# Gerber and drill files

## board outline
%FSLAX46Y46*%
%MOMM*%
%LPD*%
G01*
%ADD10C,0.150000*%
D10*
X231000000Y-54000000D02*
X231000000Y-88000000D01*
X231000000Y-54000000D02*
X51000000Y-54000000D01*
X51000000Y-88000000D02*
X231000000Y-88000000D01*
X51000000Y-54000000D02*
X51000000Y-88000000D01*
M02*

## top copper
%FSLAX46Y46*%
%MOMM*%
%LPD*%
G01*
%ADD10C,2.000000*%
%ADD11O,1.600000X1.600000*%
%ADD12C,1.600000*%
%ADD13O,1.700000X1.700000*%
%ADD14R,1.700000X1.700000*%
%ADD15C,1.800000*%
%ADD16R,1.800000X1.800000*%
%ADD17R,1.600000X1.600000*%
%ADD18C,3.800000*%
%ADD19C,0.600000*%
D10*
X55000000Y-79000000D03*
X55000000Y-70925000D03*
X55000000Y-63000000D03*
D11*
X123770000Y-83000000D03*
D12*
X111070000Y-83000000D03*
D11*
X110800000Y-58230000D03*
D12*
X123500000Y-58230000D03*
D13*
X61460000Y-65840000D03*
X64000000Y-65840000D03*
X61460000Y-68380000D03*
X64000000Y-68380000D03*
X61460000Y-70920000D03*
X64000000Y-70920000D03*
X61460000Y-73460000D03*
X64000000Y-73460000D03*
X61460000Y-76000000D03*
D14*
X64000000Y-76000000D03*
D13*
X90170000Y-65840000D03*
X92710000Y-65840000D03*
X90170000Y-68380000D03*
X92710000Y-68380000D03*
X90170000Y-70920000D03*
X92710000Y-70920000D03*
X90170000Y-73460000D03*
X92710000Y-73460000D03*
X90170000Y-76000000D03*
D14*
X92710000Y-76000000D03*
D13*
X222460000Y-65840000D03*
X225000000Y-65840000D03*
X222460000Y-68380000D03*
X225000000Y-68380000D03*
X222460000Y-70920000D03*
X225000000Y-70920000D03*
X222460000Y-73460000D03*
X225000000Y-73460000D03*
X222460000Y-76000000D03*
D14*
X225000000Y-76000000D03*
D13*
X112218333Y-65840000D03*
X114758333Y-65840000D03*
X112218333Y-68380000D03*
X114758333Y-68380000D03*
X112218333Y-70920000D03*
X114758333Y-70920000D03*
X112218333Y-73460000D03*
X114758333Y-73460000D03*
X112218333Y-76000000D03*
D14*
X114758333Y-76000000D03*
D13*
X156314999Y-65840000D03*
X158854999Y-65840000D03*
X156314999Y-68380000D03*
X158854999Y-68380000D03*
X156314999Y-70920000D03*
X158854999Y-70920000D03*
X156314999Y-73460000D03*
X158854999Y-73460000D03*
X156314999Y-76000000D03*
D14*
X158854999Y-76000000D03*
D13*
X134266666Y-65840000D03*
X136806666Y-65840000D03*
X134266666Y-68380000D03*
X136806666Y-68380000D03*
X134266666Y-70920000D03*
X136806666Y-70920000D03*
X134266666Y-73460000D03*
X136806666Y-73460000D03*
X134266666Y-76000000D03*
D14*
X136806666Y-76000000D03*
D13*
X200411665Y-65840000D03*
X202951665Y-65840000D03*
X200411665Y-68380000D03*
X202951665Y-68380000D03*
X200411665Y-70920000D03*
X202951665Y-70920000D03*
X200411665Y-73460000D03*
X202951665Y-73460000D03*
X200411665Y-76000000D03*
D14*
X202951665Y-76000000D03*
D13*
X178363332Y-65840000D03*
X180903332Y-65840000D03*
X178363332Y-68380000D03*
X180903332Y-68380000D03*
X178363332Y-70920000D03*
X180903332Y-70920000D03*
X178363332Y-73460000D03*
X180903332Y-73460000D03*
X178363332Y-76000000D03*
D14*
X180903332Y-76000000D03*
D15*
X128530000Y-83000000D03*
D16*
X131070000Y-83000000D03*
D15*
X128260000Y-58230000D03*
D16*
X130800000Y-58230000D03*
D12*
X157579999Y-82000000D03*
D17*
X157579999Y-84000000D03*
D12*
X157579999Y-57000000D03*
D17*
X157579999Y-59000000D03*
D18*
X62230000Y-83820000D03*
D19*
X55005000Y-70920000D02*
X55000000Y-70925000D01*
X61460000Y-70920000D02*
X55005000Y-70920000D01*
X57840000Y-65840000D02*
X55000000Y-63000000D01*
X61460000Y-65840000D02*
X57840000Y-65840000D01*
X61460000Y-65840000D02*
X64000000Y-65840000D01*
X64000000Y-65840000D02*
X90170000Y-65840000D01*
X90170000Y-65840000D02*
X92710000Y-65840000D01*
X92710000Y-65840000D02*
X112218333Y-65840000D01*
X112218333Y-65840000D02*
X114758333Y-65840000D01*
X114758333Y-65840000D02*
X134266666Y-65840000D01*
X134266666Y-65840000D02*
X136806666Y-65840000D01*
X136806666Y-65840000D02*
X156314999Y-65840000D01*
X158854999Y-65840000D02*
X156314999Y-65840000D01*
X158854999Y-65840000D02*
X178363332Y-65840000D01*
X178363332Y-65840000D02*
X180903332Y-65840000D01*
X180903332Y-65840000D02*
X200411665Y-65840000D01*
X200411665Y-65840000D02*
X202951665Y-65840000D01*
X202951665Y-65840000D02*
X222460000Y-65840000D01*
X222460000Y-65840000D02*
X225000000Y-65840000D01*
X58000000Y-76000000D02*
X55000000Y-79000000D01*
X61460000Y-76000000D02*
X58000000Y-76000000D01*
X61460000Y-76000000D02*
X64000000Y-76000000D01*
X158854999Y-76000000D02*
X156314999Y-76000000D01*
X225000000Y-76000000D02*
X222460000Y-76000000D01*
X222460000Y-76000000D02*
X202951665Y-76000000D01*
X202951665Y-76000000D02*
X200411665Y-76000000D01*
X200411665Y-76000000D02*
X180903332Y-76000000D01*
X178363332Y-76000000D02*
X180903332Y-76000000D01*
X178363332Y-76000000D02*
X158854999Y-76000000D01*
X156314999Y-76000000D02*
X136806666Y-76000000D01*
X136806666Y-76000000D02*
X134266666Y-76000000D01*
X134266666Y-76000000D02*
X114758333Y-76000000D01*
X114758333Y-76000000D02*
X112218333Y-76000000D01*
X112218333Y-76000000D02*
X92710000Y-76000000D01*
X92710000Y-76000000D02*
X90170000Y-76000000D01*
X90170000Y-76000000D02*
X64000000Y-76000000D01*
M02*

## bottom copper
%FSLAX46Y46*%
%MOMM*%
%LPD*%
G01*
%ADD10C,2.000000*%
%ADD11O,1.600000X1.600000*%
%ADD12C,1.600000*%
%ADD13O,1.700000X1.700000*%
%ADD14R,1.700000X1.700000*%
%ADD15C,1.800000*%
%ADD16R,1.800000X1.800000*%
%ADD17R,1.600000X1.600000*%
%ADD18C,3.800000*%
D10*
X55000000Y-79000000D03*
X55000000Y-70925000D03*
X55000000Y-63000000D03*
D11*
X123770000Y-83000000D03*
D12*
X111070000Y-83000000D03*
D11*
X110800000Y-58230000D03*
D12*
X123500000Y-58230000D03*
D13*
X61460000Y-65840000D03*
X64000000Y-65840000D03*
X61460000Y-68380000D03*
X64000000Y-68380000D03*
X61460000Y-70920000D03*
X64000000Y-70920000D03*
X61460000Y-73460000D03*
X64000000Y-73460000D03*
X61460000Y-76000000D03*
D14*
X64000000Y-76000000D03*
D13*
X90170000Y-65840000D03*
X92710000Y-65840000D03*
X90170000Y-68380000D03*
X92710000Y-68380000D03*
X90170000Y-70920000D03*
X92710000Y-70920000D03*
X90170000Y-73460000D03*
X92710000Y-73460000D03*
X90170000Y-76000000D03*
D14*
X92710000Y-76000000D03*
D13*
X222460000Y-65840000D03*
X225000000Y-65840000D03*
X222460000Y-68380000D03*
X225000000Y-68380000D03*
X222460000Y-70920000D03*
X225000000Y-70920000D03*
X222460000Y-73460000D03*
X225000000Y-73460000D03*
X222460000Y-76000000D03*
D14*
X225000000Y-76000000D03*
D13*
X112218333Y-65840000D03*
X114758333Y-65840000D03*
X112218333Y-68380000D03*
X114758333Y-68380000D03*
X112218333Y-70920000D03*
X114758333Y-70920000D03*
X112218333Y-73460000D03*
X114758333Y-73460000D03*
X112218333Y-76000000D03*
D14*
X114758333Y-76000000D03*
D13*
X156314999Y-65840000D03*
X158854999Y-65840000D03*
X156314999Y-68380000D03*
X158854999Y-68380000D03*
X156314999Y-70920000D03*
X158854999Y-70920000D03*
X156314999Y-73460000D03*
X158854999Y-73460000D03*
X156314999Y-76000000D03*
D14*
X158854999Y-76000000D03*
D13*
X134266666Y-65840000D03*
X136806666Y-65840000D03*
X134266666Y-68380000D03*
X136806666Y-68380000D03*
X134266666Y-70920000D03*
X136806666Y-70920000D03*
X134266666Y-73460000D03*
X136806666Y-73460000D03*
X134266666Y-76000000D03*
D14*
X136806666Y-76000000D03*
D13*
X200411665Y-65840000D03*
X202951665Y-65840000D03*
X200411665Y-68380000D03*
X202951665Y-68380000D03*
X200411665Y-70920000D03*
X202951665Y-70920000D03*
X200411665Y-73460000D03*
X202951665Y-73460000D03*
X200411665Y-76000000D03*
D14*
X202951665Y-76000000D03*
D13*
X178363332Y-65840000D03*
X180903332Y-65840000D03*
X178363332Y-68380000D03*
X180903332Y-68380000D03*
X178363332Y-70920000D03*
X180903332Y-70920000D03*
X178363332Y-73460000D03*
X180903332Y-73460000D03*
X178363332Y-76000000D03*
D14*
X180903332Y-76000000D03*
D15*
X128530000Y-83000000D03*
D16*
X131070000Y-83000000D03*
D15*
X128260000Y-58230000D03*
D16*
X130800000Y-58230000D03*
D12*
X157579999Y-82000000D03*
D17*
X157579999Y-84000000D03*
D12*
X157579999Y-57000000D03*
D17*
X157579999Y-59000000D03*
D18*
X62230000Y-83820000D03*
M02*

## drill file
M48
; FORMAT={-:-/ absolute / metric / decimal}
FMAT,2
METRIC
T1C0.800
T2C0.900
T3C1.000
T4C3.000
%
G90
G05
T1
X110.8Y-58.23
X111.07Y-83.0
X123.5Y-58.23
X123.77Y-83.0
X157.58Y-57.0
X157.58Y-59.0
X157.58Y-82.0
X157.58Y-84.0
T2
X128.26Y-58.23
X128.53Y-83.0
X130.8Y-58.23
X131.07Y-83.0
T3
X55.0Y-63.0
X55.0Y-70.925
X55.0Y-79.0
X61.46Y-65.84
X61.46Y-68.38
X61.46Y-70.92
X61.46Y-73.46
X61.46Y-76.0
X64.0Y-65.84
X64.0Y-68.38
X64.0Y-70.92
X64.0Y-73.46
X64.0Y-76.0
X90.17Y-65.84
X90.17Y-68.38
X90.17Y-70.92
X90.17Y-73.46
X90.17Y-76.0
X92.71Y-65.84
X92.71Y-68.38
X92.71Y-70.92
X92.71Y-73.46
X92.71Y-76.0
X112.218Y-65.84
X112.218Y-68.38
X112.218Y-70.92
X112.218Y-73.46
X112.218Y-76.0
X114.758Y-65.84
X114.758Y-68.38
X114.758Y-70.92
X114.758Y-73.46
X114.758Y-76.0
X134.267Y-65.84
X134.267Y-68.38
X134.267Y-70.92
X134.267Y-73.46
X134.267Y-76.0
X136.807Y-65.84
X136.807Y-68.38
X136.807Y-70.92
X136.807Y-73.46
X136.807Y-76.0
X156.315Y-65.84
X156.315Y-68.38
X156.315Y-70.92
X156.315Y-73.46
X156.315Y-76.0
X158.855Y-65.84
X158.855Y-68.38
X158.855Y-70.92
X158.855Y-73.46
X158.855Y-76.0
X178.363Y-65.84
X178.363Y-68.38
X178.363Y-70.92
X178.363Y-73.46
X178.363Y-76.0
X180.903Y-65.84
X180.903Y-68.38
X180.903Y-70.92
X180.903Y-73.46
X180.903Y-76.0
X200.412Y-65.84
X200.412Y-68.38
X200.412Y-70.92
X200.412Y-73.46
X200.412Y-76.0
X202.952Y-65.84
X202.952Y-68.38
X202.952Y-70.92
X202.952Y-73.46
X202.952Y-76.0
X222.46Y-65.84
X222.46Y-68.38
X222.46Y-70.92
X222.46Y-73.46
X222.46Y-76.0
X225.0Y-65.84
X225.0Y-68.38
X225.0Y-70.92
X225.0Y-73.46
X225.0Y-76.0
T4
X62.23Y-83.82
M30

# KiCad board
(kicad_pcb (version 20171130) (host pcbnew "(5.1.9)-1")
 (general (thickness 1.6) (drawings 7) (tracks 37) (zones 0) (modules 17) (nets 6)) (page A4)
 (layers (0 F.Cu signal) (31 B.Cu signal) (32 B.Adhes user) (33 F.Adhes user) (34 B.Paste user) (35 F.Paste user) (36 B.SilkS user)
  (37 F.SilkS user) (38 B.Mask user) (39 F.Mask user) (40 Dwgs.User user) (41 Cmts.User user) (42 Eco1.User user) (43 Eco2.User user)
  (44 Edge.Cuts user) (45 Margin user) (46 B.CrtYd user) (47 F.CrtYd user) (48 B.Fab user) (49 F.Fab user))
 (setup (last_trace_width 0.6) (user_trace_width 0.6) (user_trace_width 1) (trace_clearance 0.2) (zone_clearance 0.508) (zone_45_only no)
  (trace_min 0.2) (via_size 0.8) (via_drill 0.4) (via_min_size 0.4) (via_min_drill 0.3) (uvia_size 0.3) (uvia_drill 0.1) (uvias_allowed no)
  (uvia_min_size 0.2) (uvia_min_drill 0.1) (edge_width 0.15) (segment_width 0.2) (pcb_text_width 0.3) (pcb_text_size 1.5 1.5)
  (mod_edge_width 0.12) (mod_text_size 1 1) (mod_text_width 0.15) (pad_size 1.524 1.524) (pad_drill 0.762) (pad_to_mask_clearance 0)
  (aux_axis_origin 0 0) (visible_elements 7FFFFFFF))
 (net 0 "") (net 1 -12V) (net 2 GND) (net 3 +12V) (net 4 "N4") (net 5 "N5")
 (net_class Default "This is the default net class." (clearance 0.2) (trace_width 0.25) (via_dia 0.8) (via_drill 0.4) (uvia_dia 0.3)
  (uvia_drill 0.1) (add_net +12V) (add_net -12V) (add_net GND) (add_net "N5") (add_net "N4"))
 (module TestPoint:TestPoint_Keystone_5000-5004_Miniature (layer F.Cu) (at 55 79)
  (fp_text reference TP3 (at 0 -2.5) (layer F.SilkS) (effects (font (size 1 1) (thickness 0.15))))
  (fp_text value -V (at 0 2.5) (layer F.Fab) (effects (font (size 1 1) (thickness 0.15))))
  (pad 1 thru_hole circle (at 0 0) (size 2 2) (drill 1) (layers *.Cu *.Mask) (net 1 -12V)))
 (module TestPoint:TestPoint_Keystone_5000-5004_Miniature (layer F.Cu) (at 55 70.925)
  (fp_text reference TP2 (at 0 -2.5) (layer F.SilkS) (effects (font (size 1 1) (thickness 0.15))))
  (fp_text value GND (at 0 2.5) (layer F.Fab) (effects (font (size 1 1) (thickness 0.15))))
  (pad 1 thru_hole circle (at 0 0) (size 2 2) (drill 1) (layers *.Cu *.Mask) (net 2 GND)))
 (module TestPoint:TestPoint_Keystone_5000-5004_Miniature (layer F.Cu) (at 55 63)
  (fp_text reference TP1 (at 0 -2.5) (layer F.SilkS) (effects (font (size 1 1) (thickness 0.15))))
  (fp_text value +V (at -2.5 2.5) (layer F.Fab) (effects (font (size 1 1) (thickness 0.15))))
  (pad 1 thru_hole circle (at 0 0) (size 2 2) (drill 1) (layers *.Cu *.Mask) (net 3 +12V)))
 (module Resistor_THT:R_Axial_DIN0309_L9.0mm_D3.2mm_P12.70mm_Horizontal (layer F.Cu) (at 111.07 83)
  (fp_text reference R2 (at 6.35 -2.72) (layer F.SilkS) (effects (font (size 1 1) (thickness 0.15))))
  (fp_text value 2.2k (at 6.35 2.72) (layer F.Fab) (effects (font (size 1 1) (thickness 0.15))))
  (pad 2 thru_hole oval (at 12.7 0) (size 1.6 1.6) (drill 0.8) (layers *.Cu *.Mask) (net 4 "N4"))
  (pad 1 thru_hole circle (at 0 0) (size 1.6 1.6) (drill 0.8) (layers *.Cu *.Mask) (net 2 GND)))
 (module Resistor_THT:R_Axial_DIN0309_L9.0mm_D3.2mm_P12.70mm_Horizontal (layer F.Cu) (at 123.5 58.23 180)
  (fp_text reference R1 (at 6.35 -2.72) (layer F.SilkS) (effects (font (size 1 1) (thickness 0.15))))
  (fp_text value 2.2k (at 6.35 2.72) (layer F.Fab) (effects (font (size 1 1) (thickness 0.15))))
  (pad 2 thru_hole oval (at 12.7 0 180) (size 1.6 1.6) (drill 0.8) (layers *.Cu *.Mask) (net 3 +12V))
  (pad 1 thru_hole circle (at 0 0 180) (size 1.6 1.6) (drill 0.8) (layers *.Cu *.Mask) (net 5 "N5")))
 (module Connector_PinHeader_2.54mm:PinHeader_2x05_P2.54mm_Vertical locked (layer F.Cu) (at 64 76 180)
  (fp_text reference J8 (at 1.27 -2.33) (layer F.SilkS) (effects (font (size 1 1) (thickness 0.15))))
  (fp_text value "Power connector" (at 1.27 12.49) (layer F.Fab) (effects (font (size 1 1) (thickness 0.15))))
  (pad 10 thru_hole oval (at 2.54 10.16 180) (size 1.7 1.7) (drill 1) (layers *.Cu *.Mask) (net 3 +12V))
  (pad 9 thru_hole oval (at 0 10.16 180) (size 1.7 1.7) (drill 1) (layers *.Cu *.Mask) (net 3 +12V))
  (pad 8 thru_hole oval (at 2.54 7.62 180) (size 1.7 1.7) (drill 1) (layers *.Cu *.Mask) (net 2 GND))
  (pad 7 thru_hole oval (at 0 7.62 180) (size 1.7 1.7) (drill 1) (layers *.Cu *.Mask) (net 2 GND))
  (pad 6 thru_hole oval (at 2.54 5.08 180) (size 1.7 1.7) (drill 1) (layers *.Cu *.Mask) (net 2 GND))
  (pad 5 thru_hole oval (at 0 5.08 180) (size 1.7 1.7) (drill 1) (layers *.Cu *.Mask) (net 2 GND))
  (pad 4 thru_hole oval (at 2.54 2.54 180) (size 1.7 1.7) (drill 1) (layers *.Cu *.Mask) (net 2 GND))
  (pad 3 thru_hole oval (at 0 2.54 180) (size 1.7 1.7) (drill 1) (layers *.Cu *.Mask) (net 2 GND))
  (pad 2 thru_hole oval (at 2.54 0 180) (size 1.7 1.7) (drill 1) (layers *.Cu *.Mask) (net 1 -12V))
  (pad 1 thru_hole rect (at 0 0 180) (size 1.7 1.7) (drill 1) (layers *.Cu *.Mask) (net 1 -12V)))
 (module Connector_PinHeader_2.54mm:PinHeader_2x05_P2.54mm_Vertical (layer F.Cu) (at 92.71 76 180)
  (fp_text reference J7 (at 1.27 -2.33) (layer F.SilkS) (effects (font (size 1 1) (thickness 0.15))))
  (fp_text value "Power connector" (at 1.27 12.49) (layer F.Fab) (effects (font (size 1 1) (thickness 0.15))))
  (pad 10 thru_hole oval (at 2.54 10.16 180) (size 1.7 1.7) (drill 1) (layers *.Cu *.Mask) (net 3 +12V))
  (pad 9 thru_hole oval (at 0 10.16 180) (size 1.7 1.7) (drill 1) (layers *.Cu *.Mask) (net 3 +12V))
  (pad 8 thru_hole oval (at 2.54 7.62 180) (size 1.7 1.7) (drill 1) (layers *.Cu *.Mask) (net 2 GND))
  (pad 7 thru_hole oval (at 0 7.62 180) (size 1.7 1.7) (drill 1) (layers *.Cu *.Mask) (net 2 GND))
  (pad 6 thru_hole oval (at 2.54 5.08 180) (size 1.7 1.7) (drill 1) (layers *.Cu *.Mask) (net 2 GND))
  (pad 5 thru_hole oval (at 0 5.08 180) (size 1.7 1.7) (drill 1) (layers *.Cu *.Mask) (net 2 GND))
  (pad 4 thru_hole oval (at 2.54 2.54 180) (size 1.7 1.7) (drill 1) (layers *.Cu *.Mask) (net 2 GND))
  (pad 3 thru_hole oval (at 0 2.54 180) (size 1.7 1.7) (drill 1) (layers *.Cu *.Mask) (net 2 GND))
  (pad 2 thru_hole oval (at 2.54 0 180) (size 1.7 1.7) (drill 1) (layers *.Cu *.Mask) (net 1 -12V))
  (pad 1 thru_hole rect (at 0 0 180) (size 1.7 1.7) (drill 1) (layers *.Cu *.Mask) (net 1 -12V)))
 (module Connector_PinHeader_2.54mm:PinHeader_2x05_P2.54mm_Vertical (layer F.Cu) (at 225 76 180)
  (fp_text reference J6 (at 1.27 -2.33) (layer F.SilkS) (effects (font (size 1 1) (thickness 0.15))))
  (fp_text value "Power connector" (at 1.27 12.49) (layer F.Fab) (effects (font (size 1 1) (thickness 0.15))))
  (pad 10 thru_hole oval (at 2.54 10.16 180) (size 1.7 1.7) (drill 1) (layers *.Cu *.Mask) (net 3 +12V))
  (pad 9 thru_hole oval (at 0 10.16 180) (size 1.7 1.7) (drill 1) (layers *.Cu *.Mask) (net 3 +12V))
  (pad 8 thru_hole oval (at 2.54 7.62 180) (size 1.7 1.7) (drill 1) (layers *.Cu *.Mask) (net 2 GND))
  (pad 7 thru_hole oval (at 0 7.62 180) (size 1.7 1.7) (drill 1) (layers *.Cu *.Mask) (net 2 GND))
  (pad 6 thru_hole oval (at 2.54 5.08 180) (size 1.7 1.7) (drill 1) (layers *.Cu *.Mask) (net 2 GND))
  (pad 5 thru_hole oval (at 0 5.08 180) (size 1.7 1.7) (drill 1) (layers *.Cu *.Mask) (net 2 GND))
  (pad 4 thru_hole oval (at 2.54 2.54 180) (size 1.7 1.7) (drill 1) (layers *.Cu *.Mask) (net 2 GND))
  (pad 3 thru_hole oval (at 0 2.54 180) (size 1.7 1.7) (drill 1) (layers *.Cu *.Mask) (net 2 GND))
  (pad 2 thru_hole oval (at 2.54 0 180) (size 1.7 1.7) (drill 1) (layers *.Cu *.Mask) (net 1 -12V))
  (pad 1 thru_hole rect (at 0 0 180) (size 1.7 1.7) (drill 1) (layers *.Cu *.Mask) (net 1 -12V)))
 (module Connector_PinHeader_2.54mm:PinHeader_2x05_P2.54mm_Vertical (layer F.Cu) (at 114.758333 76 180)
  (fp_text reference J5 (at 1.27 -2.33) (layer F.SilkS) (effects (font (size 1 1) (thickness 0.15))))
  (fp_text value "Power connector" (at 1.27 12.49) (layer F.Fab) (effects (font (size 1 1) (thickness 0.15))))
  (pad 10 thru_hole oval (at 2.54 10.16 180) (size 1.7 1.7) (drill 1) (layers *.Cu *.Mask) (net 3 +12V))
  (pad 9 thru_hole oval (at 0 10.16 180) (size 1.7 1.7) (drill 1) (layers *.Cu *.Mask) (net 3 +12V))
  (pad 8 thru_hole oval (at 2.54 7.62 180) (size 1.7 1.7) (drill 1) (layers *.Cu *.Mask) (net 2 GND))
  (pad 7 thru_hole oval (at 0 7.62 180) (size 1.7 1.7) (drill 1) (layers *.Cu *.Mask) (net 2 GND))
  (pad 6 thru_hole oval (at 2.54 5.08 180) (size 1.7 1.7) (drill 1) (layers *.Cu *.Mask) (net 2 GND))
  (pad 5 thru_hole oval (at 0 5.08 180) (size 1.7 1.7) (drill 1) (layers *.Cu *.Mask) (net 2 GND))
  (pad 4 thru_hole oval (at 2.54 2.54 180) (size 1.7 1.7) (drill 1) (layers *.Cu *.Mask) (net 2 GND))
  (pad 3 thru_hole oval (at 0 2.54 180) (size 1.7 1.7) (drill 1) (layers *.Cu *.Mask) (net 2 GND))
  (pad 2 thru_hole oval (at 2.54 0 180) (size 1.7 1.7) (drill 1) (layers *.Cu *.Mask) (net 1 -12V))
  (pad 1 thru_hole rect (at 0 0 180) (size 1.7 1.7) (drill 1) (layers *.Cu *.Mask) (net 1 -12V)))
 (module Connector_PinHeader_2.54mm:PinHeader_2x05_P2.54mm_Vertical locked (layer F.Cu) (at 158.854999 76 180)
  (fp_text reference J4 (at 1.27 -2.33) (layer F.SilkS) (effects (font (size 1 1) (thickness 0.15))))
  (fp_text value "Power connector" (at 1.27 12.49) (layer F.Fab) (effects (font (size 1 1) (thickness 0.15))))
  (pad 10 thru_hole oval (at 2.54 10.16 180) (size 1.7 1.7) (drill 1) (layers *.Cu *.Mask) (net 3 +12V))
  (pad 9 thru_hole oval (at 0 10.16 180) (size 1.7 1.7) (drill 1) (layers *.Cu *.Mask) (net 3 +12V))
  (pad 8 thru_hole oval (at 2.54 7.62 180) (size 1.7 1.7) (drill 1) (layers *.Cu *.Mask) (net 2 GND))
  (pad 7 thru_hole oval (at 0 7.62 180) (size 1.7 1.7) (drill 1) (layers *.Cu *.Mask) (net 2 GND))
  (pad 6 thru_hole oval (at 2.54 5.08 180) (size 1.7 1.7) (drill 1) (layers *.Cu *.Mask) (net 2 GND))
  (pad 5 thru_hole oval (at 0 5.08 180) (size 1.7 1.7) (drill 1) (layers *.Cu *.Mask) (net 2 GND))
  (pad 4 thru_hole oval (at 2.54 2.54 180) (size 1.7 1.7) (drill 1) (layers *.Cu *.Mask) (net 2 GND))
  (pad 3 thru_hole oval (at 0 2.54 180) (size 1.7 1.7) (drill 1) (layers *.Cu *.Mask) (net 2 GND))
  (pad 2 thru_hole oval (at 2.54 0 180) (size 1.7 1.7) (drill 1) (layers *.Cu *.Mask) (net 1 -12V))
  (pad 1 thru_hole rect (at 0 0 180) (size 1.7 1.7) (drill 1) (layers *.Cu *.Mask) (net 1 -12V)))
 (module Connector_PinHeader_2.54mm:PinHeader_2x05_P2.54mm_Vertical (layer F.Cu) (at 136.806666 76 180)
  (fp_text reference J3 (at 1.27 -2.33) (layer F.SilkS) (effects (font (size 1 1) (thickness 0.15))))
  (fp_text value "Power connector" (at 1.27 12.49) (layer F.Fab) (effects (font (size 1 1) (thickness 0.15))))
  (pad 10 thru_hole oval (at 2.54 10.16 180) (size 1.7 1.7) (drill 1) (layers *.Cu *.Mask) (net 3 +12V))
  (pad 9 thru_hole oval (at 0 10.16 180) (size 1.7 1.7) (drill 1) (layers *.Cu *.Mask) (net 3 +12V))
  (pad 8 thru_hole oval (at 2.54 7.62 180) (size 1.7 1.7) (drill 1) (layers *.Cu *.Mask) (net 2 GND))
  (pad 7 thru_hole oval (at 0 7.62 180) (size 1.7 1.7) (drill 1) (layers *.Cu *.Mask) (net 2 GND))
  (pad 6 thru_hole oval (at 2.54 5.08 180) (size 1.7 1.7) (drill 1) (layers *.Cu *.Mask) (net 2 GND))
  (pad 5 thru_hole oval (at 0 5.08 180) (size 1.7 1.7) (drill 1) (layers *.Cu *.Mask) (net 2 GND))
  (pad 4 thru_hole oval (at 2.54 2.54 180) (size 1.7 1.7) (drill 1) (layers *.Cu *.Mask) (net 2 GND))
  (pad 3 thru_hole oval (at 0 2.54 180) (size 1.7 1.7) (drill 1) (layers *.Cu *.Mask) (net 2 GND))
  (pad 2 thru_hole oval (at 2.54 0 180) (size 1.7 1.7) (drill 1) (layers *.Cu *.Mask) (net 1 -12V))
  (pad 1 thru_hole rect (at 0 0 180) (size 1.7 1.7) (drill 1) (layers *.Cu *.Mask) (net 1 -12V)))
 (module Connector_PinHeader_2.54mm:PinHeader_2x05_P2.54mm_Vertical (layer F.Cu) (at 202.951665 76 180)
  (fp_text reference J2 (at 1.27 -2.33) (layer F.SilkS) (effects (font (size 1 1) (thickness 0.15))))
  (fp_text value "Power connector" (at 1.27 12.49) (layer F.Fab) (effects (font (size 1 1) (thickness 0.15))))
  (pad 10 thru_hole oval (at 2.54 10.16 180) (size 1.7 1.7) (drill 1) (layers *.Cu *.Mask) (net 3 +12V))
  (pad 9 thru_hole oval (at 0 10.16 180) (size 1.7 1.7) (drill 1) (layers *.Cu *.Mask) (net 3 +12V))
  (pad 8 thru_hole oval (at 2.54 7.62 180) (size 1.7 1.7) (drill 1) (layers *.Cu *.Mask) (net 2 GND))
  (pad 7 thru_hole oval (at 0 7.62 180) (size 1.7 1.7) (drill 1) (layers *.Cu *.Mask) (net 2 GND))
  (pad 6 thru_hole oval (at 2.54 5.08 180) (size 1.7 1.7) (drill 1) (layers *.Cu *.Mask) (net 2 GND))
  (pad 5 thru_hole oval (at 0 5.08 180) (size 1.7 1.7) (drill 1) (layers *.Cu *.Mask) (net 2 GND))
  (pad 4 thru_hole oval (at 2.54 2.54 180) (size 1.7 1.7) (drill 1) (layers *.Cu *.Mask) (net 2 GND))
  (pad 3 thru_hole oval (at 0 2.54 180) (size 1.7 1.7) (drill 1) (layers *.Cu *.Mask) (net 2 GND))
  (pad 2 thru_hole oval (at 2.54 0 180) (size 1.7 1.7) (drill 1) (layers *.Cu *.Mask) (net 1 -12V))
  (pad 1 thru_hole rect (at 0 0 180) (size 1.7 1.7) (drill 1) (layers *.Cu *.Mask) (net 1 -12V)))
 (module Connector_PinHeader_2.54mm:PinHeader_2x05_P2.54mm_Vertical (layer F.Cu) (at 180.903332 76 180)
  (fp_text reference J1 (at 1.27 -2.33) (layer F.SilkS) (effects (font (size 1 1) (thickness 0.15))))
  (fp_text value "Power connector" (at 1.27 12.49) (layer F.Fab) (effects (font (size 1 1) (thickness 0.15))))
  (pad 10 thru_hole oval (at 2.54 10.16 180) (size 1.7 1.7) (drill 1) (layers *.Cu *.Mask) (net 3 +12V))
  (pad 9 thru_hole oval (at 0 10.16 180) (size 1.7 1.7) (drill 1) (layers *.Cu *.Mask) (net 3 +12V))
  (pad 8 thru_hole oval (at 2.54 7.62 180) (size 1.7 1.7) (drill 1) (layers *.Cu *.Mask) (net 2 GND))
  (pad 7 thru_hole oval (at 0 7.62 180) (size 1.7 1.7) (drill 1) (layers *.Cu *.Mask) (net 2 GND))
  (pad 6 thru_hole oval (at 2.54 5.08 180) (size 1.7 1.7) (drill 1) (layers *.Cu *.Mask) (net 2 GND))
  (pad 5 thru_hole oval (at 0 5.08 180) (size 1.7 1.7) (drill 1) (layers *.Cu *.Mask) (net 2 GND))
  (pad 4 thru_hole oval (at 2.54 2.54 180) (size 1.7 1.7) (drill 1) (layers *.Cu *.Mask) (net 2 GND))
  (pad 3 thru_hole oval (at 0 2.54 180) (size 1.7 1.7) (drill 1) (layers *.Cu *.Mask) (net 2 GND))
  (pad 2 thru_hole oval (at 2.54 0 180) (size 1.7 1.7) (drill 1) (layers *.Cu *.Mask) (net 1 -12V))
  (pad 1 thru_hole rect (at 0 0 180) (size 1.7 1.7) (drill 1) (layers *.Cu *.Mask) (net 1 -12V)))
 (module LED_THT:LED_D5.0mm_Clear (layer F.Cu) (at 131.07 83 180)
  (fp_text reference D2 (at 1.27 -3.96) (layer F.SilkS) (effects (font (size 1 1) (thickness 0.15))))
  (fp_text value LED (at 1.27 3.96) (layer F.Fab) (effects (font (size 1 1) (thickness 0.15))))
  (pad 2 thru_hole circle (at 2.54 0 180) (size 1.8 1.8) (drill 0.9) (layers *.Cu *.Mask) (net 4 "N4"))
  (pad 1 thru_hole rect (at 0 0 180) (size 1.8 1.8) (drill 0.9) (layers *.Cu *.Mask) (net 1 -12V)))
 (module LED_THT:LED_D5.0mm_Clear (layer F.Cu) (at 130.8 58.23 180)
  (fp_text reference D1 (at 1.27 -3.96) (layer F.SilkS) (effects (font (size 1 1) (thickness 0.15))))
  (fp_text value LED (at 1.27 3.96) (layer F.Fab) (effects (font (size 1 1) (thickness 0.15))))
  (pad 2 thru_hole circle (at 2.54 0 180) (size 1.8 1.8) (drill 0.9) (layers *.Cu *.Mask) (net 5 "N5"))
  (pad 1 thru_hole rect (at 0 0 180) (size 1.8 1.8) (drill 0.9) (layers *.Cu *.Mask) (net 2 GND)))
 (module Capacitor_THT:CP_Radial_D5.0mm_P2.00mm (layer F.Cu) (at 157.579999 84 90)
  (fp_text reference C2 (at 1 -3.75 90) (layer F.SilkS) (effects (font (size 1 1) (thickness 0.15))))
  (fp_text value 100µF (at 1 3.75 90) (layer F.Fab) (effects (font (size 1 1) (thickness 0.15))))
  (pad 2 thru_hole circle (at 2 0 90) (size 1.6 1.6) (drill 0.8) (layers *.Cu *.Mask) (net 1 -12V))
  (pad 1 thru_hole rect (at 0 0 90) (size 1.6 1.6) (drill 0.8) (layers *.Cu *.Mask) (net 2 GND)))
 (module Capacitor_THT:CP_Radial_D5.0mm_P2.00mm (layer F.Cu) (at 157.579999 59 90)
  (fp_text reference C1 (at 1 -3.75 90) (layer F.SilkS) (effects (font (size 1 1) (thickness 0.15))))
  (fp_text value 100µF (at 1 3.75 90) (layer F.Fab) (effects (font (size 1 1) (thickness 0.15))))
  (pad 2 thru_hole circle (at 2 0 90) (size 1.6 1.6) (drill 0.8) (layers *.Cu *.Mask) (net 2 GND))
  (pad 1 thru_hole rect (at 0 0 90) (size 1.6 1.6) (drill 0.8) (layers *.Cu *.Mask) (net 3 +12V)))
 (gr_line (start 231 54) (end 231 88) (layer Edge.Cuts) (width 0.15))
 (gr_line (start 231 54) (end 51 54) (layer Edge.Cuts) (width 0.15))
 (gr_line (start 51 88) (end 231 88) (layer Edge.Cuts) (width 0.15))
 (gr_line (start 51 54) (end 51 88) (layer Edge.Cuts) (width 0.15))
 (via (at 62.23 83.82) (size 3.8) (drill 3) (layers F.Cu B.Cu) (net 2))
 (segment (start 55.005 70.92) (end 55 70.925) (width 0.6) (layer F.Cu) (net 2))
 (segment (start 61.46 70.92) (end 55.005 70.92) (width 0.6) (layer F.Cu) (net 2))
 (segment (start 57.84 65.84) (end 55 63) (width 0.6) (layer F.Cu) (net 3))
 (segment (start 61.46 65.84) (end 57.84 65.84) (width 0.6) (layer F.Cu) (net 3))
 (segment (start 61.46 65.84) (end 64 65.84) (width 0.6) (layer F.Cu) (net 3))
 (segment (start 64 65.84) (end 90.17 65.84) (width 0.6) (layer F.Cu) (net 3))
 (segment (start 90.17 65.84) (end 92.71 65.84) (width 0.6) (layer F.Cu) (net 3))
 (segment (start 92.71 65.84) (end 112.218333 65.84) (width 0.6) (layer F.Cu) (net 3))
 (segment (start 112.218333 65.84) (end 114.758333 65.84) (width 0.6) (layer F.Cu) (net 3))
 (segment (start 114.758333 65.84) (end 134.266666 65.84) (width 0.6) (layer F.Cu) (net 3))
 (segment (start 134.266666 65.84) (end 136.806666 65.84) (width 0.6) (layer F.Cu) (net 3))
 (segment (start 136.806666 65.84) (end 156.314999 65.84) (width 0.6) (layer F.Cu) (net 3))
 (segment (start 158.854999 65.84) (end 156.314999 65.84) (width 0.6) (layer F.Cu) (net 3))
 (segment (start 158.854999 65.84) (end 178.363332 65.84) (width 0.6) (layer F.Cu) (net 3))
 (segment (start 178.363332 65.84) (end 180.903332 65.84) (width 0.6) (layer F.Cu) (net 3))
 (segment (start 180.903332 65.84) (end 200.411665 65.84) (width 0.6) (layer F.Cu) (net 3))
 (segment (start 200.411665 65.84) (end 202.951665 65.84) (width 0.6) (layer F.Cu) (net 3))
 (segment (start 202.951665 65.84) (end 222.46 65.84) (width 0.6) (layer F.Cu) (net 3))
 (segment (start 222.46 65.84) (end 225 65.84) (width 0.6) (layer F.Cu) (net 3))
 (segment (start 58 76) (end 55 79) (width 0.6) (layer F.Cu) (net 1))
 (segment (start 61.46 76) (end 58 76) (width 0.6) (layer F.Cu) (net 1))
 (segment (start 61.46 76) (end 64 76) (width 0.6) (layer F.Cu) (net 1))
 (segment (start 158.854999 76) (end 156.314999 76) (width 0.6) (layer F.Cu) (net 1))
 (segment (start 225 76) (end 222.46 76) (width 0.6) (layer F.Cu) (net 1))
 (segment (start 222.46 76) (end 202.951665 76) (width 0.6) (layer F.Cu) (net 1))
 (segment (start 202.951665 76) (end 200.411665 76) (width 0.6) (layer F.Cu) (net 1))
 (segment (start 200.411665 76) (end 180.903332 76) (width 0.6) (layer F.Cu) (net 1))
 (segment (start 178.363332 76) (end 180.903332 76) (width 0.6) (layer F.Cu) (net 1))
 (segment (start 178.363332 76) (end 158.854999 76) (width 0.6) (layer F.Cu) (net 1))
 (segment (start 156.314999 76) (end 136.806666 76) (width 0.6) (layer F.Cu) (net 1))
 (segment (start 136.806666 76) (end 134.266666 76) (width 0.6) (layer F.Cu) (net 1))
 (segment (start 134.266666 76) (end 114.758333 76) (width 0.6) (layer F.Cu) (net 1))
 (segment (start 114.758333 76) (end 112.218333 76) (width 0.6) (layer F.Cu) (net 1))
 (segment (start 112.218333 76) (end 92.71 76) (width 0.6) (layer F.Cu) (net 1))
 (segment (start 92.71 76) (end 90.17 76) (width 0.6) (layer F.Cu) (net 1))
 (segment (start 90.17 76) (end 64 76) (width 0.6) (layer F.Cu) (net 1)))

